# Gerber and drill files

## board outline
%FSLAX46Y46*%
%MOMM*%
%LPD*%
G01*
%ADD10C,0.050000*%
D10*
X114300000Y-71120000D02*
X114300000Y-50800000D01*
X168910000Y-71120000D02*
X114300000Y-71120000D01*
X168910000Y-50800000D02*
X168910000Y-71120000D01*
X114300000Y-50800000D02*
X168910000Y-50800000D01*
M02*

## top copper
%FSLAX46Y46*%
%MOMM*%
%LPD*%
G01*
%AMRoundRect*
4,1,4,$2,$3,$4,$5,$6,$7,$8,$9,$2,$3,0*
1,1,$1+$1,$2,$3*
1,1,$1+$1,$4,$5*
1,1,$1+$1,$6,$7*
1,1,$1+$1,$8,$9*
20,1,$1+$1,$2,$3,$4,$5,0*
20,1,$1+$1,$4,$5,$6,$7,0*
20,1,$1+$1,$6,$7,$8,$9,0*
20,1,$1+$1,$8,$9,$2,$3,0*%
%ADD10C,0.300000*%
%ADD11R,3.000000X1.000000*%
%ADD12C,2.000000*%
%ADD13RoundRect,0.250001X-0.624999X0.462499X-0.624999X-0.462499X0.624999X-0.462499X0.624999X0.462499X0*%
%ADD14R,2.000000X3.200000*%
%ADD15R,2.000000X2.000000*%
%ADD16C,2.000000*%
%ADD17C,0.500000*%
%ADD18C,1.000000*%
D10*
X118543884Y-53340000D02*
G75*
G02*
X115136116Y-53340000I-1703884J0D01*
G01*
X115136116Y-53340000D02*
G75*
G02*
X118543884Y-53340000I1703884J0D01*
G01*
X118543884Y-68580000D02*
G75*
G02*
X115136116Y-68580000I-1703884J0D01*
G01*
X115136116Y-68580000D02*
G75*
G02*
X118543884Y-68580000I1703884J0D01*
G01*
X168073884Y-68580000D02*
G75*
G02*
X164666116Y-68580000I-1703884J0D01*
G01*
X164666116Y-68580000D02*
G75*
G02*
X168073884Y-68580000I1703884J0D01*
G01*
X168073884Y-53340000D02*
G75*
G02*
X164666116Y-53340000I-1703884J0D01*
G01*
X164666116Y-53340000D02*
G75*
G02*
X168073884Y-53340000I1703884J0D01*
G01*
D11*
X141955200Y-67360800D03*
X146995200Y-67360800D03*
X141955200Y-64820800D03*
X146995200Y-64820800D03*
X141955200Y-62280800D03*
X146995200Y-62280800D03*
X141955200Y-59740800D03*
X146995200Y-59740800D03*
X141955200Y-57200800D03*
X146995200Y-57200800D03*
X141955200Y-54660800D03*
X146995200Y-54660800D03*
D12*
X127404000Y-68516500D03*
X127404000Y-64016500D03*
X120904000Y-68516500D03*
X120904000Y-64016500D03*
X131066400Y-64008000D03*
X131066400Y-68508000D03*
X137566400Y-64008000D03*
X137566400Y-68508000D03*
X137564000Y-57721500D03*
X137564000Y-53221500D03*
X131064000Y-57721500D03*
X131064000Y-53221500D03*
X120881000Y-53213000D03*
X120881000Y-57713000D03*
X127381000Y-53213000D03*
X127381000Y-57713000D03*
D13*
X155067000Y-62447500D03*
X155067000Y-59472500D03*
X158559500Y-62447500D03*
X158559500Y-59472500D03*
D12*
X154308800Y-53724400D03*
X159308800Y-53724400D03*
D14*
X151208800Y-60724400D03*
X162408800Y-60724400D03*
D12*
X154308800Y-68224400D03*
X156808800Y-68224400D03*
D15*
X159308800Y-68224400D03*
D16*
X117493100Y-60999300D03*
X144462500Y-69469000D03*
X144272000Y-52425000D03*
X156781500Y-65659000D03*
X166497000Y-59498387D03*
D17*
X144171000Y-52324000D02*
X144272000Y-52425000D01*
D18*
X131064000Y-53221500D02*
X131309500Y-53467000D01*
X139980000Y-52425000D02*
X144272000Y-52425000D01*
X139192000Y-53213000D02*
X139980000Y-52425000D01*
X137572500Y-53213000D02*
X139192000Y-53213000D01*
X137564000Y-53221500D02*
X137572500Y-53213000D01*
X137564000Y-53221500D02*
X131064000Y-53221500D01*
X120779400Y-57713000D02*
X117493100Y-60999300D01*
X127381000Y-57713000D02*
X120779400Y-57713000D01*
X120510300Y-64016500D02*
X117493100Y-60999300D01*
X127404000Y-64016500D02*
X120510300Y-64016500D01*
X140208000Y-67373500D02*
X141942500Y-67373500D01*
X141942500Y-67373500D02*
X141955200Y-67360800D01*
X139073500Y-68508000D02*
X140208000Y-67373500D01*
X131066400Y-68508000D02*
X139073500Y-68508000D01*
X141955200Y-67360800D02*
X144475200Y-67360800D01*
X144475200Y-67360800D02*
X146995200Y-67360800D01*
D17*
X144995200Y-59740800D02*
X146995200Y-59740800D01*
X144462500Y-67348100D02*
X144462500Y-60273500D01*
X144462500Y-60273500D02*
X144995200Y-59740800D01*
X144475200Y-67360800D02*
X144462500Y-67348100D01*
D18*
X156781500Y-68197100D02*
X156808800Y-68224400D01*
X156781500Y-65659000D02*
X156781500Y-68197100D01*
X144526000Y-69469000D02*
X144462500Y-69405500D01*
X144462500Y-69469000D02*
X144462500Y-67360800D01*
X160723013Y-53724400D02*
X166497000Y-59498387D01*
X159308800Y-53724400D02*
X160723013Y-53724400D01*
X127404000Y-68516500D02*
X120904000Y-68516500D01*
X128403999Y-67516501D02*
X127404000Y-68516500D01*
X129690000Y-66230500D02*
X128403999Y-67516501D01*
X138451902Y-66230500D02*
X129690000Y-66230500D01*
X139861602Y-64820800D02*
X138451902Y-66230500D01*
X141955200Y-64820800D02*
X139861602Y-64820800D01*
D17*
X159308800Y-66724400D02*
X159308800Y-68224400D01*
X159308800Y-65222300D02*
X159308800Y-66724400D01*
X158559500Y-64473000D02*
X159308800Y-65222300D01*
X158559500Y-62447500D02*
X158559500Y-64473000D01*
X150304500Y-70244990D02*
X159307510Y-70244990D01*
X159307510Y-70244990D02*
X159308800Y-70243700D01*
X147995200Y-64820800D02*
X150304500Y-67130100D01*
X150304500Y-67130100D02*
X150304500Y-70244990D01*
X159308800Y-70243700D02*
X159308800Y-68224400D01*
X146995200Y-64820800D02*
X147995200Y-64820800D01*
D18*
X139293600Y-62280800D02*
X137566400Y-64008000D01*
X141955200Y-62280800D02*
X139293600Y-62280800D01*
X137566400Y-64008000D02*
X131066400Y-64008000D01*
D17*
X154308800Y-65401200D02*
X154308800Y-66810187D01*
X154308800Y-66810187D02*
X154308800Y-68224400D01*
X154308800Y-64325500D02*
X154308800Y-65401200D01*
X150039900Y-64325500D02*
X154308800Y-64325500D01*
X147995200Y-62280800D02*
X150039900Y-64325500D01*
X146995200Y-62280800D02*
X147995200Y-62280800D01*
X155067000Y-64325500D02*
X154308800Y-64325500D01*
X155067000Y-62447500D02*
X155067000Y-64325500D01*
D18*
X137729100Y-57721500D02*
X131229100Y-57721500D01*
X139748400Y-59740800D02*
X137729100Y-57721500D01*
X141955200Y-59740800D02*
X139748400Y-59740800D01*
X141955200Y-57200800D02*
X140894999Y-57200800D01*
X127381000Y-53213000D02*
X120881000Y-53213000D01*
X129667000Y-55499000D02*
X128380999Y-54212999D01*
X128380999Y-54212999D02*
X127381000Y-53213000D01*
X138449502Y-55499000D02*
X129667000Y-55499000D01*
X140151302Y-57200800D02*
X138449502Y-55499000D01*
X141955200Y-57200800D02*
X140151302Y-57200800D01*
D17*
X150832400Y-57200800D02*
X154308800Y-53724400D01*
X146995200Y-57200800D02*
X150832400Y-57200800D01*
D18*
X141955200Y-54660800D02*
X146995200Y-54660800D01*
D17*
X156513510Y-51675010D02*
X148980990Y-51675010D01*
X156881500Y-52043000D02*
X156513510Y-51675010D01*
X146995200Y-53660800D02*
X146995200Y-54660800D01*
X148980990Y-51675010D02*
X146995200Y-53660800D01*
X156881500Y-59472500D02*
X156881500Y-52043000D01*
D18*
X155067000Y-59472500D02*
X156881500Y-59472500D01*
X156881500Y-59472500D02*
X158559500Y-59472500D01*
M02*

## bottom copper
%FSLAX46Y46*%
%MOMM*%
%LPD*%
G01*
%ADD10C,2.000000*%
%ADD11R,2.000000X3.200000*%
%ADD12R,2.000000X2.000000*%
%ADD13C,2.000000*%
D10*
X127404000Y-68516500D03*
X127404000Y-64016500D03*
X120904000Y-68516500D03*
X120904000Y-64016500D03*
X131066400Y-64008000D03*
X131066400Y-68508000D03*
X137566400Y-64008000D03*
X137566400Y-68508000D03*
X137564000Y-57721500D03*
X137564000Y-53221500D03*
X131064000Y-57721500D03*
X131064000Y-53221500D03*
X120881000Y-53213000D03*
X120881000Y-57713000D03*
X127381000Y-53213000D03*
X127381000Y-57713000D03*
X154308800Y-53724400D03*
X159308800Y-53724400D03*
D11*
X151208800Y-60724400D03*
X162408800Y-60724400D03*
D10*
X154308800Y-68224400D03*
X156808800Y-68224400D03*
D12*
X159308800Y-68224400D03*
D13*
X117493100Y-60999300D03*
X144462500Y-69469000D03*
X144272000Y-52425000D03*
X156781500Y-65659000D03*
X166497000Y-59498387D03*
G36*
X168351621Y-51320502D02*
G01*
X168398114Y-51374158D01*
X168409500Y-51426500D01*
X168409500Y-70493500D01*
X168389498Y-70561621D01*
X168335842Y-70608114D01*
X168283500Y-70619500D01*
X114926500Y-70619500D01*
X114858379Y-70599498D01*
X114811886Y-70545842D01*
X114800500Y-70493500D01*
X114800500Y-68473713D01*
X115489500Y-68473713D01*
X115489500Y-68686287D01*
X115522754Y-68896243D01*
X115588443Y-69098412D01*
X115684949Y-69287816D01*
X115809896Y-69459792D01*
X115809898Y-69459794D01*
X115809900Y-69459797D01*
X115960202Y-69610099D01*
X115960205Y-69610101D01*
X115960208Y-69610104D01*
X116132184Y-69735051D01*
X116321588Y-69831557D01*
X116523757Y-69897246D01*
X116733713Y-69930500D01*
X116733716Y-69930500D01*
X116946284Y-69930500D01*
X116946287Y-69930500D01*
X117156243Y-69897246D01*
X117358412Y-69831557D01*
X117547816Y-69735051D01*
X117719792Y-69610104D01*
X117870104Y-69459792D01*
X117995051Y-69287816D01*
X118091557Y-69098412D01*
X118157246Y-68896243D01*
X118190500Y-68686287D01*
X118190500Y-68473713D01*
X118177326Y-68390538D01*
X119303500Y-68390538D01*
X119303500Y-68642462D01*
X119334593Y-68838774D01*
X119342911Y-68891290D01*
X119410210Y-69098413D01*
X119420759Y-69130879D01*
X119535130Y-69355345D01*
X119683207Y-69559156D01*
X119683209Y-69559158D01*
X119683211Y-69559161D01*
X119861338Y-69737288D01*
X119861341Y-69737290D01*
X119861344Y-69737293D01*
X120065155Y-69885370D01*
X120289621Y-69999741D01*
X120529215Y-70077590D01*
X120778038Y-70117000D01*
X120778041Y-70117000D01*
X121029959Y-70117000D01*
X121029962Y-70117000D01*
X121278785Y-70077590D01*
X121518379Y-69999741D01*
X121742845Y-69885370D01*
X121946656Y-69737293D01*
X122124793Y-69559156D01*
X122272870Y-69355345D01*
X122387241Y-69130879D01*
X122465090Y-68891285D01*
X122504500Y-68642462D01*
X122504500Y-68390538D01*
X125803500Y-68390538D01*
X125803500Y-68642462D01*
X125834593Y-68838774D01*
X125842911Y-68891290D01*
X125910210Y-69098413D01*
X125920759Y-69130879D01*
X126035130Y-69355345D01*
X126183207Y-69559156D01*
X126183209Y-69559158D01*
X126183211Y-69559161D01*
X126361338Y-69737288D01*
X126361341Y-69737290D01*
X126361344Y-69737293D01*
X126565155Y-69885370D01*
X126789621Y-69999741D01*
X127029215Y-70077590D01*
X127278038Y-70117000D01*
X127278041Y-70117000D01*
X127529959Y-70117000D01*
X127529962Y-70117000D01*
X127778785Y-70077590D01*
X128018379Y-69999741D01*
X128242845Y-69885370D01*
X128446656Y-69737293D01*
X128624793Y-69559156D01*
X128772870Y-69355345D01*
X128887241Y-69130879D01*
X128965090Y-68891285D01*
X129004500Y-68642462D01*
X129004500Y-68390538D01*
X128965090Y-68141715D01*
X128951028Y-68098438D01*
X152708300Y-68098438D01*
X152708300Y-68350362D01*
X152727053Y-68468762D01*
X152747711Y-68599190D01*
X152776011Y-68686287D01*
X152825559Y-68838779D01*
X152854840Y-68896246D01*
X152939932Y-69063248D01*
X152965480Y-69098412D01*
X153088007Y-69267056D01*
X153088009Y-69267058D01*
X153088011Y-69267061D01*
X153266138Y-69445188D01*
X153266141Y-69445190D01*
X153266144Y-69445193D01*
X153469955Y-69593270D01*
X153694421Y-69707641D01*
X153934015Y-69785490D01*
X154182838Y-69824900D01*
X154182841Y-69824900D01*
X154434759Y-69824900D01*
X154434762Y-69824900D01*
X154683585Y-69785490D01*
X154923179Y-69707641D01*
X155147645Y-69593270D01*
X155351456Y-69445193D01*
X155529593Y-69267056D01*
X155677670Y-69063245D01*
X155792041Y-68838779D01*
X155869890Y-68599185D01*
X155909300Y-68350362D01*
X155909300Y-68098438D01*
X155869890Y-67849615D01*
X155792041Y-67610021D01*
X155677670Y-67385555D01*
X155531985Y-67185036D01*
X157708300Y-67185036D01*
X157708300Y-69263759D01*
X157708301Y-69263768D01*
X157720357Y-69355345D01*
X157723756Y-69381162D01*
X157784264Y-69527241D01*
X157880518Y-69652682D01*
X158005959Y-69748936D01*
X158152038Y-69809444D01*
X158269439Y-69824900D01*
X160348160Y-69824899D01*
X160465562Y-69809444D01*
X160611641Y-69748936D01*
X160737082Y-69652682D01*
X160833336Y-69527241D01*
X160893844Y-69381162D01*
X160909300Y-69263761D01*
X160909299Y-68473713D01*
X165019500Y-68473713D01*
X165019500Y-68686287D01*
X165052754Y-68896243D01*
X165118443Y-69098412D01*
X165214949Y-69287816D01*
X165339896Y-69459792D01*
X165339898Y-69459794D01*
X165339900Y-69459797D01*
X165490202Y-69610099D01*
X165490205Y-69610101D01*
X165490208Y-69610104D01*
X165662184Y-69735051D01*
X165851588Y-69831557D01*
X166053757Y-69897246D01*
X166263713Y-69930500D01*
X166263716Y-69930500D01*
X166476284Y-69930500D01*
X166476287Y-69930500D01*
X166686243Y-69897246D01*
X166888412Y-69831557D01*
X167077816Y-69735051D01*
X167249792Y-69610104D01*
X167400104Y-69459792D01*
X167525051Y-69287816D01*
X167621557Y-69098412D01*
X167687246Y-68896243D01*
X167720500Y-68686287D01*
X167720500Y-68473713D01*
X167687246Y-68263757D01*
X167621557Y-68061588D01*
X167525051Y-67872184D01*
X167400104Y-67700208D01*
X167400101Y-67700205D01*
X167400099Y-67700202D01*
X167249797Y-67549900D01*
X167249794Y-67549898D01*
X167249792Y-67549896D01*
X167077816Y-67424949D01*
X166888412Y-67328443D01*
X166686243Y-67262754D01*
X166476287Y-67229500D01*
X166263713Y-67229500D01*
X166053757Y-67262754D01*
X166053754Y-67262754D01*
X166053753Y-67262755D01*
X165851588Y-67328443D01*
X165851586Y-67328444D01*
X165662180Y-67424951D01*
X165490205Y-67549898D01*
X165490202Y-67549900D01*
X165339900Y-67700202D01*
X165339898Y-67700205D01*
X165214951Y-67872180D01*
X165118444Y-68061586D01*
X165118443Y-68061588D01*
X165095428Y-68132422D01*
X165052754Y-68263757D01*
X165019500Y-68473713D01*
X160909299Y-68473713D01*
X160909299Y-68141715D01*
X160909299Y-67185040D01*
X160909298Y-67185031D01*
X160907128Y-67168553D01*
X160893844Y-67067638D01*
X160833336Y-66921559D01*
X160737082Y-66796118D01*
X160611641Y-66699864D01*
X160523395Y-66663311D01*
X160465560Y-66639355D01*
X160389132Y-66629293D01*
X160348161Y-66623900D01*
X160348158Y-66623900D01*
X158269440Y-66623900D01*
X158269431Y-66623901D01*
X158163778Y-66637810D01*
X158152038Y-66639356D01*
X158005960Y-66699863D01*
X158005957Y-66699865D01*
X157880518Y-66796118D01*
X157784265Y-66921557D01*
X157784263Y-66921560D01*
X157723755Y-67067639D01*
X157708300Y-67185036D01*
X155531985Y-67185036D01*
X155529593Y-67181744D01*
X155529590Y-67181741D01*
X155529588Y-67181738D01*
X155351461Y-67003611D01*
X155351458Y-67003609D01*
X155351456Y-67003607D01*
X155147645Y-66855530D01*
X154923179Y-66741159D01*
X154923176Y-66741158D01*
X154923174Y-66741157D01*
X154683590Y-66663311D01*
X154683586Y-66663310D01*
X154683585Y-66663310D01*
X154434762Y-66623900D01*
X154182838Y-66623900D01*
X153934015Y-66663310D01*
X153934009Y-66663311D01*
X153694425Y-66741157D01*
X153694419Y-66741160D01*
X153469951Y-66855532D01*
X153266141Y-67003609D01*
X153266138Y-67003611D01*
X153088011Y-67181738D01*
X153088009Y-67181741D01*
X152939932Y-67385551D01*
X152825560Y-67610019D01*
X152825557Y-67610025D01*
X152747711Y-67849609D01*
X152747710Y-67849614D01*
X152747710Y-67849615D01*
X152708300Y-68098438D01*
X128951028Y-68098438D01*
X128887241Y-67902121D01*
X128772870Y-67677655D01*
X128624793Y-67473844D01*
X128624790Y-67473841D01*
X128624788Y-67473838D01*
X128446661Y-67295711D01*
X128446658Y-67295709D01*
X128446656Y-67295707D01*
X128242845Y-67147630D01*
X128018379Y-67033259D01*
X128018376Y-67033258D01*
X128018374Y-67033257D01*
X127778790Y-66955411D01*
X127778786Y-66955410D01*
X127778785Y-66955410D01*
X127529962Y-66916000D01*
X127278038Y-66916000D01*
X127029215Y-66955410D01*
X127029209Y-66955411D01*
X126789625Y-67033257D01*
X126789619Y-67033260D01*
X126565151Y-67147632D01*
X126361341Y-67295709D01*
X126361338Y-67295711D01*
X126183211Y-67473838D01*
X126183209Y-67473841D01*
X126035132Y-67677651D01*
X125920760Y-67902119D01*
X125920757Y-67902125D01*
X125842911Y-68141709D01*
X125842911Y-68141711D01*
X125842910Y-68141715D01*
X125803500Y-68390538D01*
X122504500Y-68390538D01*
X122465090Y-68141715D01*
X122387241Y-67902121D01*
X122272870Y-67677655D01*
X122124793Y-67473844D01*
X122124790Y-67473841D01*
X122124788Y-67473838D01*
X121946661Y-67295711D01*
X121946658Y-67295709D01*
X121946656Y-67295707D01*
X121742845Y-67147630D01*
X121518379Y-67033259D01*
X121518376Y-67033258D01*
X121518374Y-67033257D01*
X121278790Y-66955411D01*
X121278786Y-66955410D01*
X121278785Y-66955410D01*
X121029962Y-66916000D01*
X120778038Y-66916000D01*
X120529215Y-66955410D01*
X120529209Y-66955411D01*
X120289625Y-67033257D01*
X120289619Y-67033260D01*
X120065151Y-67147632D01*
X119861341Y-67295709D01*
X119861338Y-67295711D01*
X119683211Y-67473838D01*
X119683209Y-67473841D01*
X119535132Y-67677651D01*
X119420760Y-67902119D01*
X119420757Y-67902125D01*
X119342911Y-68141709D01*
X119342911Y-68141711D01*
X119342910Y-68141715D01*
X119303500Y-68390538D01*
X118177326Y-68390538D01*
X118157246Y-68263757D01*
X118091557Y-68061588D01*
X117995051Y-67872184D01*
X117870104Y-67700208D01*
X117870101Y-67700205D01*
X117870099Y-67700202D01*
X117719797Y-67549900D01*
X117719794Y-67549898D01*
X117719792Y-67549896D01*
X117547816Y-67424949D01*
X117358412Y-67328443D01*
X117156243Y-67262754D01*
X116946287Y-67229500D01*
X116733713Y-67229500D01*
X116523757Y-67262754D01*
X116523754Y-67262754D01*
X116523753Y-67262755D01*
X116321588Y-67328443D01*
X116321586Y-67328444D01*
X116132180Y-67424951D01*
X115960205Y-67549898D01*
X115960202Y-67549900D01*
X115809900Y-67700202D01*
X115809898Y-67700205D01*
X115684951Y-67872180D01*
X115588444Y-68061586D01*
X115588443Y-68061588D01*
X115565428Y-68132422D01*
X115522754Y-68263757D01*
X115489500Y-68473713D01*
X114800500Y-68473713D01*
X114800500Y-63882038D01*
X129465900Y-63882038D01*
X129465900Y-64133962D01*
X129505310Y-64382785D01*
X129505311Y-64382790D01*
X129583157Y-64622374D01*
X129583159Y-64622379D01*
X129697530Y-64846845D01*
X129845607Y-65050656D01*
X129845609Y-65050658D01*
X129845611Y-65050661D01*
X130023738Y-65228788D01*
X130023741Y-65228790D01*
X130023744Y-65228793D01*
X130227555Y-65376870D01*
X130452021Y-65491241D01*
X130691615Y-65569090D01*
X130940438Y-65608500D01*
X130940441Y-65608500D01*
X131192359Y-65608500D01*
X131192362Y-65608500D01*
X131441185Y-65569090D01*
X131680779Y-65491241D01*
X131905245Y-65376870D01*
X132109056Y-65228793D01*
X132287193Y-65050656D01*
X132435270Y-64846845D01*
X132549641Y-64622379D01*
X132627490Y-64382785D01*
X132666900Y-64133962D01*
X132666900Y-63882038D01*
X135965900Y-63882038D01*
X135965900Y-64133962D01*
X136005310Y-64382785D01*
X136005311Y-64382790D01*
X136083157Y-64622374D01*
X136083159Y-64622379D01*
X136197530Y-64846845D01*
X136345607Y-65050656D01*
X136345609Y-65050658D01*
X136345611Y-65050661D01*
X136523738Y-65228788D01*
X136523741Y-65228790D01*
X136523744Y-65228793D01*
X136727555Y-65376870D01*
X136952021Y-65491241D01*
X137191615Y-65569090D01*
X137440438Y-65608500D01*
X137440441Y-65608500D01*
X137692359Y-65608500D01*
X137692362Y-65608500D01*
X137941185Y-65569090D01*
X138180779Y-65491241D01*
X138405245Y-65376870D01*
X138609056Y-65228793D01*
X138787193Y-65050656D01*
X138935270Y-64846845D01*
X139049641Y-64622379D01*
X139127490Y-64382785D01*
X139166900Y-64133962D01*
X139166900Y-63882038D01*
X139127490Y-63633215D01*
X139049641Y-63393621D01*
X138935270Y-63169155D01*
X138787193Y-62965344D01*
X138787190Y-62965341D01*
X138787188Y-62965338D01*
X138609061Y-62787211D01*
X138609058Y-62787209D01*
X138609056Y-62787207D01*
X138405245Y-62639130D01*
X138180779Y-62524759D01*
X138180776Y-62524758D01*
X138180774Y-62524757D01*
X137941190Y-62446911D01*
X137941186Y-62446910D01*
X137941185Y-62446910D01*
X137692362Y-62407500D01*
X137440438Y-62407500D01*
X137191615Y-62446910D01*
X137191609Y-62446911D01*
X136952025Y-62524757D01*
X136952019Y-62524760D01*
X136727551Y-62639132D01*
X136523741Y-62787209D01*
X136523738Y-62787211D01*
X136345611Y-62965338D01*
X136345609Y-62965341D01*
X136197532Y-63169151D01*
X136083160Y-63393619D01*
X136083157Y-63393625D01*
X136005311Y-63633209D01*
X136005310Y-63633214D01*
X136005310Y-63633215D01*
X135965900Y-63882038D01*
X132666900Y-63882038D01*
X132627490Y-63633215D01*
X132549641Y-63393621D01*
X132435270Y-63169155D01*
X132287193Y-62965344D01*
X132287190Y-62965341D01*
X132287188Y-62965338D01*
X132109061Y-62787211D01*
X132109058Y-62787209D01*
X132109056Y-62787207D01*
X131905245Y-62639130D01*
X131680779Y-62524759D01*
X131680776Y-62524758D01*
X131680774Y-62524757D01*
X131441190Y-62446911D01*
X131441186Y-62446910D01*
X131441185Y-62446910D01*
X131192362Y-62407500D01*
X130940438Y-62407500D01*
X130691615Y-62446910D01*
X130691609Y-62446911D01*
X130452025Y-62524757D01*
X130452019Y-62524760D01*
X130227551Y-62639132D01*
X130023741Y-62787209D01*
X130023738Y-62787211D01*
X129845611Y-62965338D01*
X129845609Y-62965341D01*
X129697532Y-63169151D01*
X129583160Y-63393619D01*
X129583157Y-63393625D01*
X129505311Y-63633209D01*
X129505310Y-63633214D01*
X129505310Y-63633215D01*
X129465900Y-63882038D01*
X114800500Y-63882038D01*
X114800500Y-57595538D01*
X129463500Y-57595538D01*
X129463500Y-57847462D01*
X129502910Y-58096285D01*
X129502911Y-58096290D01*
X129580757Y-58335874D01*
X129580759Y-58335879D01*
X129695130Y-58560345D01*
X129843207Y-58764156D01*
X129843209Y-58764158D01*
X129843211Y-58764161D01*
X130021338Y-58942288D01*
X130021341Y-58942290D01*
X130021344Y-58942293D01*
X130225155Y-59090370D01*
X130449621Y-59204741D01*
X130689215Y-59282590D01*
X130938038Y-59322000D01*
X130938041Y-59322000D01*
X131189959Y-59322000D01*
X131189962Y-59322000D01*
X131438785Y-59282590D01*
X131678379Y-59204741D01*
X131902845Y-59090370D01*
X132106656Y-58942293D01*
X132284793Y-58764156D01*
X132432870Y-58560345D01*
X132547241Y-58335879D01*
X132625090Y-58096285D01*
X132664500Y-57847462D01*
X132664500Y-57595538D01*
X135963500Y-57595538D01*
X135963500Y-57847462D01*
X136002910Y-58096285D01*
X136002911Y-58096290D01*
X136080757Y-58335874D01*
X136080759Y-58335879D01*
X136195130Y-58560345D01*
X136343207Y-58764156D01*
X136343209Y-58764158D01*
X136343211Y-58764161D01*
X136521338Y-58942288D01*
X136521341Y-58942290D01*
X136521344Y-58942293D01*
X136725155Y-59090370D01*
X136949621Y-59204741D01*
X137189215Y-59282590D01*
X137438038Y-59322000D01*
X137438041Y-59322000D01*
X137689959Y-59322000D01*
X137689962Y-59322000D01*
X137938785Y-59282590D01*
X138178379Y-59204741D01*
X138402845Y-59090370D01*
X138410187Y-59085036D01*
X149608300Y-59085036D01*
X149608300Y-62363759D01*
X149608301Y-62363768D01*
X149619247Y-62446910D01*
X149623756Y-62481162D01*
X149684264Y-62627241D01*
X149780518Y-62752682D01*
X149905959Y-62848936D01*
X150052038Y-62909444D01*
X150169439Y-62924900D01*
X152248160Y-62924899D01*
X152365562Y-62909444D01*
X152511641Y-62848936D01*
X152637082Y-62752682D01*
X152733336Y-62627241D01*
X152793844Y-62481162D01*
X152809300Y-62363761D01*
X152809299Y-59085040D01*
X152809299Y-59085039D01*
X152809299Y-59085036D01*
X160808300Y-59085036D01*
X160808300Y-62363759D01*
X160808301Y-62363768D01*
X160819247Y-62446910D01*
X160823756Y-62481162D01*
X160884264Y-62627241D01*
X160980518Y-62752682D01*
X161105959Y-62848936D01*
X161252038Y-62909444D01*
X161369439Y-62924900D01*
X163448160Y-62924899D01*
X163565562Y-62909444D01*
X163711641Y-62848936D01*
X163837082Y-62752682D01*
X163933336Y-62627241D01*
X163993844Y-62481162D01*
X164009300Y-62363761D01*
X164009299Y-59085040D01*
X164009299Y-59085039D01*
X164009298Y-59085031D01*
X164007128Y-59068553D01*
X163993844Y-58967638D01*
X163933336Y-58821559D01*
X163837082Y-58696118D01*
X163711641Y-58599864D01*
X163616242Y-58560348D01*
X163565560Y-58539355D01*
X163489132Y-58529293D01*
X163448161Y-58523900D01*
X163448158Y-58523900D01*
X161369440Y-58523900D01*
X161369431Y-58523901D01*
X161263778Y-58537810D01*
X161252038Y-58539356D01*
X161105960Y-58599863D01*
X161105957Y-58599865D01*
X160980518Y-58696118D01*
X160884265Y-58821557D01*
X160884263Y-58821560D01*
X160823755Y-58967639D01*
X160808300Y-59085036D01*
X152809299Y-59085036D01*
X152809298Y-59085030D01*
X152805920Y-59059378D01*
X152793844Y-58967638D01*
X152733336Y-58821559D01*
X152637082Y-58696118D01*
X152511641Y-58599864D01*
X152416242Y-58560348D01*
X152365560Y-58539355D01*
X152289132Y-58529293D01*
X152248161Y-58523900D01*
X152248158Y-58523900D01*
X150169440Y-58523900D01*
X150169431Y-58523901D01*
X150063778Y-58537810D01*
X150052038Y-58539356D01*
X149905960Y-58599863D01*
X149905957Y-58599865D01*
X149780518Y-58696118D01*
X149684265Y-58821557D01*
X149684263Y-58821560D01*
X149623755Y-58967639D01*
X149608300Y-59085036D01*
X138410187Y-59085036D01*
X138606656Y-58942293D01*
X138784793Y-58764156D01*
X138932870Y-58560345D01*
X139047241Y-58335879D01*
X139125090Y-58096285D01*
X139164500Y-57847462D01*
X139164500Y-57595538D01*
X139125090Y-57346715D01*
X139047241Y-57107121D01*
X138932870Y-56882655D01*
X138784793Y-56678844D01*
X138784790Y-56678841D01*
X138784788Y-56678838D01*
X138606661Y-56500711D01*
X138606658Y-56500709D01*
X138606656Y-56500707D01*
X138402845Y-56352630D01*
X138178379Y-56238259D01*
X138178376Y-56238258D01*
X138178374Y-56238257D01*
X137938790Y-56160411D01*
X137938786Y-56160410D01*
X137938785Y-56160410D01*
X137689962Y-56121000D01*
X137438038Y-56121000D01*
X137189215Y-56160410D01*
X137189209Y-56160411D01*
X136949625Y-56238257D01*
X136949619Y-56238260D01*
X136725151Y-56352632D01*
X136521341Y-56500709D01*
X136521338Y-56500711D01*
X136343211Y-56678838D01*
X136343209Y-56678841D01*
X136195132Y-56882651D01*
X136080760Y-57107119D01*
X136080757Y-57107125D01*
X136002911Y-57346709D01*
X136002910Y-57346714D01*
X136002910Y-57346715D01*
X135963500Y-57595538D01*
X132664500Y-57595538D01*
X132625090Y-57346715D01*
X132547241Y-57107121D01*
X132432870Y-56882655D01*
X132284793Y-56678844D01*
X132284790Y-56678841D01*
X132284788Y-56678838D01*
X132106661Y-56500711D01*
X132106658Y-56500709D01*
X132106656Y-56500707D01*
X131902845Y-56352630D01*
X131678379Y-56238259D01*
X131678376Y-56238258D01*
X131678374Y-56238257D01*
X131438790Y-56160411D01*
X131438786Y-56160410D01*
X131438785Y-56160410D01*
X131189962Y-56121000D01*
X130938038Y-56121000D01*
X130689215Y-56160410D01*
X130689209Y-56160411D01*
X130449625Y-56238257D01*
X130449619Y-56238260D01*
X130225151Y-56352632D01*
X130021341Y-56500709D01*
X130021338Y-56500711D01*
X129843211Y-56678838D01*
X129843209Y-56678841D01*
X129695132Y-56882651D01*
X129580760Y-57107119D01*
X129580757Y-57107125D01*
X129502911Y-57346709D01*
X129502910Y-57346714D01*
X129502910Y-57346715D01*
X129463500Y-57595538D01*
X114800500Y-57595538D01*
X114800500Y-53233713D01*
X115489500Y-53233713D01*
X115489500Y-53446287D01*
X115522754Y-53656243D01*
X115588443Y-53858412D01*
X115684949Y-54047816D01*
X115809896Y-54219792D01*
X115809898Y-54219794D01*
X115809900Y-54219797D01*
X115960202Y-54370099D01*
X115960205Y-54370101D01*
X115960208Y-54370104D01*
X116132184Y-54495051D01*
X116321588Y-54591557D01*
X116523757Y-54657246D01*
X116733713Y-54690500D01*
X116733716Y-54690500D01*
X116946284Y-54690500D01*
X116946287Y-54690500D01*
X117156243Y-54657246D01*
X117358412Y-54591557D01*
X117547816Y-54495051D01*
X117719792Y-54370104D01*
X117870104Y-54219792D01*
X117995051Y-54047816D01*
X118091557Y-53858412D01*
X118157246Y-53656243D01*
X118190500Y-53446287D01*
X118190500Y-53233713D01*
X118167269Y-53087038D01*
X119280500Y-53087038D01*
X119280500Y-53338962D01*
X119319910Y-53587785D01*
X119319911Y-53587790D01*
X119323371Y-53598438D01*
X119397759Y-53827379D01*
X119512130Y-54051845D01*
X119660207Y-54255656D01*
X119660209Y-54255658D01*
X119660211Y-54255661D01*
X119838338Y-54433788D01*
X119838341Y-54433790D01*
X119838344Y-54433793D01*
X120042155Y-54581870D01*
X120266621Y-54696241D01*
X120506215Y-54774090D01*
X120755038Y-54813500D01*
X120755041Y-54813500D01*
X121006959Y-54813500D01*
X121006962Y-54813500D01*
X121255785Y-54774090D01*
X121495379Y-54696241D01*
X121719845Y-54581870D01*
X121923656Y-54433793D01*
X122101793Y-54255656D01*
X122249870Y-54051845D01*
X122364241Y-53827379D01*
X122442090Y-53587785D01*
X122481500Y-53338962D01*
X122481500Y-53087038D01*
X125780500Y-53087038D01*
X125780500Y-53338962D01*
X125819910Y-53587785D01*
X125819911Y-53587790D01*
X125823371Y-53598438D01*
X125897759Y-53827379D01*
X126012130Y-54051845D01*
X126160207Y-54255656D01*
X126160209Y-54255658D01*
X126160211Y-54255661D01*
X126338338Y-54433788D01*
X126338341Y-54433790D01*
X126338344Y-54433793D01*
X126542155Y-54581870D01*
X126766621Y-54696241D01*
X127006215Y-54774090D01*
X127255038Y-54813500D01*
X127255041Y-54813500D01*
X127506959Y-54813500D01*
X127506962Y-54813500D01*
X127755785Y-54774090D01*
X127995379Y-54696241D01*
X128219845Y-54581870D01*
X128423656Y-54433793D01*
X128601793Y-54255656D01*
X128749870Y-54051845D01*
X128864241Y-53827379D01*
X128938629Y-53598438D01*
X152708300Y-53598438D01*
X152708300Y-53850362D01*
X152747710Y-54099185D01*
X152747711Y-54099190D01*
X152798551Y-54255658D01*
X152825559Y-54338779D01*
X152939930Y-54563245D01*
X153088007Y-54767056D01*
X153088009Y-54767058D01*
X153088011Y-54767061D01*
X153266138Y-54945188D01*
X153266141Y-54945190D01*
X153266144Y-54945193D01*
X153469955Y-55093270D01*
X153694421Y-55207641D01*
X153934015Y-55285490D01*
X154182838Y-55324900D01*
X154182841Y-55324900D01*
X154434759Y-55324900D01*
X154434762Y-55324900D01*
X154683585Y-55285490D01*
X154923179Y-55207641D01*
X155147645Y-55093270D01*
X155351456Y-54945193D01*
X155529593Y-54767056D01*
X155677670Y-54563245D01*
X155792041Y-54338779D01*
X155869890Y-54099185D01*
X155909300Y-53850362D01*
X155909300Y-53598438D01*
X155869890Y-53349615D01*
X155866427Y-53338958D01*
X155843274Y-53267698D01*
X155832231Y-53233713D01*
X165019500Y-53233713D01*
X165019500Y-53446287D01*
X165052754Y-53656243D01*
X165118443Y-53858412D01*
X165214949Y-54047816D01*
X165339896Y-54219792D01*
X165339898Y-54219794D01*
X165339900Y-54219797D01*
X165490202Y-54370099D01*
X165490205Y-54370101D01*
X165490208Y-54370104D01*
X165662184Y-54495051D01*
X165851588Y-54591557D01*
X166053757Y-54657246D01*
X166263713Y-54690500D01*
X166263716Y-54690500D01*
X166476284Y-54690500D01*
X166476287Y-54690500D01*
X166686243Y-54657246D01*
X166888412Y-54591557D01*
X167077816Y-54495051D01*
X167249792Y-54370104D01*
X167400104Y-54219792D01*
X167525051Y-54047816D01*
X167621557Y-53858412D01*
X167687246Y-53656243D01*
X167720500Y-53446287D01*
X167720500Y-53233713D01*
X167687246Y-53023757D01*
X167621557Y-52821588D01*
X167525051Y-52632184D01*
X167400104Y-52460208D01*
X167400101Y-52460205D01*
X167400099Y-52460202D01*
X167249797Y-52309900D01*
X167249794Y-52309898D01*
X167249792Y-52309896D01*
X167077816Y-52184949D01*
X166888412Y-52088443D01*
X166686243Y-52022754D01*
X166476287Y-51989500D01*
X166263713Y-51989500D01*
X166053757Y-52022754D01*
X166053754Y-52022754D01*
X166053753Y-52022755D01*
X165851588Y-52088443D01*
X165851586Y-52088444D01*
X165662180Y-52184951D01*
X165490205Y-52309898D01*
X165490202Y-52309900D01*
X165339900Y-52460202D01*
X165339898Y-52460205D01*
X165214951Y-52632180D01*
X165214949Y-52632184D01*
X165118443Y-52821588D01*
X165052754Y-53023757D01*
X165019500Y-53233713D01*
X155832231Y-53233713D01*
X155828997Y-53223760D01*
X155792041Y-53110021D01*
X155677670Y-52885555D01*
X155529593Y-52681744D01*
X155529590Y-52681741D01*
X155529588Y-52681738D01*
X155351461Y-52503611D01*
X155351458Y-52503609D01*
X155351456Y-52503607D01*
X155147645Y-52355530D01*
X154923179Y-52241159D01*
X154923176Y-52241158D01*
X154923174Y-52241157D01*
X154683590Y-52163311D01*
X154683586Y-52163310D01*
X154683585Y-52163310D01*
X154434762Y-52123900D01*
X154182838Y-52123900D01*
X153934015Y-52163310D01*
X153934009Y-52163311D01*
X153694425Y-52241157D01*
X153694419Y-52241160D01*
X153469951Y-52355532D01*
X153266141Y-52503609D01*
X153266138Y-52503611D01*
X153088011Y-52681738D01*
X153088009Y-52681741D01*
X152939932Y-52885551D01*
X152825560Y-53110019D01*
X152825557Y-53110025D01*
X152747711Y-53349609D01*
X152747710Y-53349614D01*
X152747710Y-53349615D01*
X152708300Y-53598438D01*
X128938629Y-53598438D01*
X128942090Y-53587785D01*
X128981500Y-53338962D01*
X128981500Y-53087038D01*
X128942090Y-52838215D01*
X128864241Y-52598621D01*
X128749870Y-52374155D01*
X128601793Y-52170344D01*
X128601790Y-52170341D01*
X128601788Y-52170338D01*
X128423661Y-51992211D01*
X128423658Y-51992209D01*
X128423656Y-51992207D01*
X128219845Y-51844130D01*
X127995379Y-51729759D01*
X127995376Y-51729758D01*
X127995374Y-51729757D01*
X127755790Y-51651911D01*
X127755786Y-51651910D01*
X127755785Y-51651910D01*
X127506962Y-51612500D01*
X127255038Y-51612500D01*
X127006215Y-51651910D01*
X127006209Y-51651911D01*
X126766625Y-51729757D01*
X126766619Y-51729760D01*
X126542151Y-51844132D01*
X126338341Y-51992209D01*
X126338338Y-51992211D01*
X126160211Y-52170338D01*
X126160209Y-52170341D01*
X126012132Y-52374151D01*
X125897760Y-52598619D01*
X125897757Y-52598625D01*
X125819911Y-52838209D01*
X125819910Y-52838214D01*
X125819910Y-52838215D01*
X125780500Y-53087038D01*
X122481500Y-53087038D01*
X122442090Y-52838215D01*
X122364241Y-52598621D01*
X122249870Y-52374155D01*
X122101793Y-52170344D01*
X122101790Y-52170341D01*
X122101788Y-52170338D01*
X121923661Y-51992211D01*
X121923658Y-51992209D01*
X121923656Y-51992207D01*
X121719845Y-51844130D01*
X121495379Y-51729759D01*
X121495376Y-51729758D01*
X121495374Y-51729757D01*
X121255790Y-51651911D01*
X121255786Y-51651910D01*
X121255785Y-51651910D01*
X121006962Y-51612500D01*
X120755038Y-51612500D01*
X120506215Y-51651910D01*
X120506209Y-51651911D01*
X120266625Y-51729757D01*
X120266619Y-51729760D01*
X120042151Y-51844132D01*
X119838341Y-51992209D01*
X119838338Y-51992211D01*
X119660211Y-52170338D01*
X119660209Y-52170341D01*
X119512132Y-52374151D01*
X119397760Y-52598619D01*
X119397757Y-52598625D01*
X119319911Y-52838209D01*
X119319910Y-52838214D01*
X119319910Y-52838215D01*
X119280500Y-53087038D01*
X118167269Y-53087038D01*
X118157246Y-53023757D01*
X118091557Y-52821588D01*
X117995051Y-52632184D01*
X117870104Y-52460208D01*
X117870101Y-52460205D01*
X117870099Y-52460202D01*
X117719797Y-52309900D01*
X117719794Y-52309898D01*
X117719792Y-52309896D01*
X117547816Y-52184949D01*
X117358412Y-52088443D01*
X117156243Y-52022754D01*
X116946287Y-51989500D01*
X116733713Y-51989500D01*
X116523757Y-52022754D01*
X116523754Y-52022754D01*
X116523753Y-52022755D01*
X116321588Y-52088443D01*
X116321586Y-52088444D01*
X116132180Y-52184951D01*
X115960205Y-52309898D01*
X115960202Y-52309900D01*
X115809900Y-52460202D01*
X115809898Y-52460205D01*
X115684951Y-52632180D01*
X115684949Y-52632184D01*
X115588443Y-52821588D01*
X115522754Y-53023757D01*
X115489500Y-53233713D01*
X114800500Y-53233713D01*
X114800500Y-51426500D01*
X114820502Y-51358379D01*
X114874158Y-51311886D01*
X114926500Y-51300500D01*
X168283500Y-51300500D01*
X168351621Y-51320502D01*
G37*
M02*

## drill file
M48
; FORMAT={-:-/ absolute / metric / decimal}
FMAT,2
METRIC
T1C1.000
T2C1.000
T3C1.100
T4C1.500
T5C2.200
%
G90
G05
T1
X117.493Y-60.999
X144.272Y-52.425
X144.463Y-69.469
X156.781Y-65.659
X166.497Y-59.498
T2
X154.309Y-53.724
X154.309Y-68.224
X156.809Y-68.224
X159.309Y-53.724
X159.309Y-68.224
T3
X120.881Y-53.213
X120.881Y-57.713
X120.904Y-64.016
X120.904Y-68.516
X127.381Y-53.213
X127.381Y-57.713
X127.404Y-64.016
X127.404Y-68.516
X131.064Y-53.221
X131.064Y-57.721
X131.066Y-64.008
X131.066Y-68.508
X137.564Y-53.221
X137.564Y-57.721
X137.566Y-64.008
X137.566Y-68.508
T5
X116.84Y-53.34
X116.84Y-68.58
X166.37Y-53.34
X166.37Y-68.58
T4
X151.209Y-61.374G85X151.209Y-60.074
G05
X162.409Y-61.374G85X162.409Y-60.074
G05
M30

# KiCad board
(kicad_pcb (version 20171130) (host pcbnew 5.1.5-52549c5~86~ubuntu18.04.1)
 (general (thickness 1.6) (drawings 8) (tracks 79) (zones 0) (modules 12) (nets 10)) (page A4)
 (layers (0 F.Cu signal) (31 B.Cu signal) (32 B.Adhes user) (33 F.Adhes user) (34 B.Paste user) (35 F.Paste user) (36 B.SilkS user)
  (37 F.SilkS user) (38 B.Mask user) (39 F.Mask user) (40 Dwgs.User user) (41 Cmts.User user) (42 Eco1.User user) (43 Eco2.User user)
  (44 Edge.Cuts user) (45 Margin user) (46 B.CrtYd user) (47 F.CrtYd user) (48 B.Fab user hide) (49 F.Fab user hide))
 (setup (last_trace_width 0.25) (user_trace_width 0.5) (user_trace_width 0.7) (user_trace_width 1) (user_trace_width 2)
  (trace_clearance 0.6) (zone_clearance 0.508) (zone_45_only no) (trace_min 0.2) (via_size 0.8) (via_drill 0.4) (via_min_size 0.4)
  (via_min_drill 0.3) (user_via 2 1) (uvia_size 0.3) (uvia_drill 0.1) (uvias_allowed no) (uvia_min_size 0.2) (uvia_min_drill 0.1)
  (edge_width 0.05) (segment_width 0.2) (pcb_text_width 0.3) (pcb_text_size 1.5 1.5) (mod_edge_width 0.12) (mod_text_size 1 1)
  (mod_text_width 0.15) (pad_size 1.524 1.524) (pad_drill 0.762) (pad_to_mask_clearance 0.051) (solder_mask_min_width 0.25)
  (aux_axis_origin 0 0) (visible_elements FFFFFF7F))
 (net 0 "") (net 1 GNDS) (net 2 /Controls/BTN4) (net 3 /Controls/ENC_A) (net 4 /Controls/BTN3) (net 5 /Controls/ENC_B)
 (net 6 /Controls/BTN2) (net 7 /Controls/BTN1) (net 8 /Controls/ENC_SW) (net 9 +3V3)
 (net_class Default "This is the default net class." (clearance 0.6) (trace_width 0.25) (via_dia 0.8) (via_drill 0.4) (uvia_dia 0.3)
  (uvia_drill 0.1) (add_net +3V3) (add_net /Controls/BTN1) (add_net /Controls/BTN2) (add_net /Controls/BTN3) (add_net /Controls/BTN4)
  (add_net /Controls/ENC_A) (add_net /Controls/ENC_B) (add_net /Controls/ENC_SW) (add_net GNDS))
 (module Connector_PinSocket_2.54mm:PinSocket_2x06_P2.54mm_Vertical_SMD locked (layer F.Cu) (at 144.4752 61.0108)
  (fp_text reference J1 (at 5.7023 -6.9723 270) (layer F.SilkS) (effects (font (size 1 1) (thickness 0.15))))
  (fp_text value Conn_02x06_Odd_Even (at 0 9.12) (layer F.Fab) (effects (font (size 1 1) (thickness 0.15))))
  (pad 12 smd rect (at -2.52 6.35) (size 3 1) (layers F.Cu F.Paste F.Mask) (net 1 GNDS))
  (pad 11 smd rect (at 2.52 6.35) (size 3 1) (layers F.Cu F.Paste F.Mask) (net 1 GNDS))
  (pad 10 smd rect (at -2.52 3.81) (size 3 1) (layers F.Cu F.Paste F.Mask) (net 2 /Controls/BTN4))
  (pad 9 smd rect (at 2.52 3.81) (size 3 1) (layers F.Cu F.Paste F.Mask) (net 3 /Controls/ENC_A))
  (pad 8 smd rect (at -2.52 1.27) (size 3 1) (layers F.Cu F.Paste F.Mask) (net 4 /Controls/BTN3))
  (pad 7 smd rect (at 2.52 1.27) (size 3 1) (layers F.Cu F.Paste F.Mask) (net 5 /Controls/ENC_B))
  (pad 6 smd rect (at -2.52 -1.27) (size 3 1) (layers F.Cu F.Paste F.Mask) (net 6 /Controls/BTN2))
  (pad 5 smd rect (at 2.52 -1.27) (size 3 1) (layers F.Cu F.Paste F.Mask) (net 1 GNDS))
  (pad 4 smd rect (at -2.52 -3.81) (size 3 1) (layers F.Cu F.Paste F.Mask) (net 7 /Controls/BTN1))
  (pad 3 smd rect (at 2.52 -3.81) (size 3 1) (layers F.Cu F.Paste F.Mask) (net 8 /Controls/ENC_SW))
  (pad 2 smd rect (at -2.52 -6.35) (size 3 1) (layers F.Cu F.Paste F.Mask) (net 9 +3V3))
  (pad 1 smd rect (at 2.52 -6.35) (size 3 1) (layers F.Cu F.Paste F.Mask) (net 9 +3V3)))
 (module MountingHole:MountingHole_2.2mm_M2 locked (layer F.Cu) (at 166.37 53.34)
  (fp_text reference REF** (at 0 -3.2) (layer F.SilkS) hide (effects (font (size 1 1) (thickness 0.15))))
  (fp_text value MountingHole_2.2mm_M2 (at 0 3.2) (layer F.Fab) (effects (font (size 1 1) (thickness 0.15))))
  (pad 1 np_thru_hole circle (at 0 0) (size 2.2 2.2) (drill 2.2) (layers *.Cu *.Mask)))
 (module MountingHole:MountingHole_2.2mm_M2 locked (layer F.Cu) (at 166.37 68.58)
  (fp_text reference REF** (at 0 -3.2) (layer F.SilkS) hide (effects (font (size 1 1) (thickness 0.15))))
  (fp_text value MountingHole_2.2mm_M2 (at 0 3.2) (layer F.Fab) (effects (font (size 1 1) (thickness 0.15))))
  (pad 1 np_thru_hole circle (at 0 0) (size 2.2 2.2) (drill 2.2) (layers *.Cu *.Mask)))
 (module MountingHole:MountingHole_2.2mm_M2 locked (layer F.Cu) (at 116.84 68.58)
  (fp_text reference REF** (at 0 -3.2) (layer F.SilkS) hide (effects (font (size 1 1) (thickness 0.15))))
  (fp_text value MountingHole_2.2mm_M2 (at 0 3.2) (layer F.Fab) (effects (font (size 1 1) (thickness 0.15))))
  (pad 1 np_thru_hole circle (at 0 0) (size 2.2 2.2) (drill 2.2) (layers *.Cu *.Mask)))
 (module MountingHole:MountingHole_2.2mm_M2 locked (layer F.Cu) (at 116.84 53.34)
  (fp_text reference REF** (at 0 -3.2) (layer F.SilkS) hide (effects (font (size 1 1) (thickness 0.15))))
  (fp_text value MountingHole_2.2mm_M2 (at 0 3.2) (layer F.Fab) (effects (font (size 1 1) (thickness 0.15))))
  (pad 1 np_thru_hole circle (at 0 0) (size 2.2 2.2) (drill 2.2) (layers *.Cu *.Mask)))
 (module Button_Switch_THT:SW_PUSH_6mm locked (layer B.Cu) (at 120.904 68.5165)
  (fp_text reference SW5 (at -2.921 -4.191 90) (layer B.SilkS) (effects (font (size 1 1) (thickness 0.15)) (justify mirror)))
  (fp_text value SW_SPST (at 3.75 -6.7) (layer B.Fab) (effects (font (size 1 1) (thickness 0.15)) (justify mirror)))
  (pad 1 thru_hole circle (at 6.5 0 270) (size 2 2) (drill 1.1) (layers *.Cu *.Mask) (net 2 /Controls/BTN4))
  (pad 2 thru_hole circle (at 6.5 -4.5 270) (size 2 2) (drill 1.1) (layers *.Cu *.Mask) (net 1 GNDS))
  (pad 1 thru_hole circle (at 0 0 270) (size 2 2) (drill 1.1) (layers *.Cu *.Mask) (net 2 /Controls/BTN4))
  (pad 2 thru_hole circle (at 0 -4.5 270) (size 2 2) (drill 1.1) (layers *.Cu *.Mask) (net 1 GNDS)))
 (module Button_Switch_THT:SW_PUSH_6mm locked (layer B.Cu) (at 137.5664 64.008 180)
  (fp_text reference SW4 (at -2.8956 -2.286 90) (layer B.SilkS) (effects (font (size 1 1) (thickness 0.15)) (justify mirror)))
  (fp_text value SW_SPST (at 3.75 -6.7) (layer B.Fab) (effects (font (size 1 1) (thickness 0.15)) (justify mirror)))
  (pad 1 thru_hole circle (at 6.5 0 90) (size 2 2) (drill 1.1) (layers *.Cu *.Mask) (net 4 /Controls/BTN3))
  (pad 2 thru_hole circle (at 6.5 -4.5 90) (size 2 2) (drill 1.1) (layers *.Cu *.Mask) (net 1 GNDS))
  (pad 1 thru_hole circle (at 0 0 90) (size 2 2) (drill 1.1) (layers *.Cu *.Mask) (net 4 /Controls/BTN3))
  (pad 2 thru_hole circle (at 0 -4.5 90) (size 2 2) (drill 1.1) (layers *.Cu *.Mask) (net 1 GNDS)))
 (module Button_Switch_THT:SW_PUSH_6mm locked (layer B.Cu) (at 131.064 57.7215)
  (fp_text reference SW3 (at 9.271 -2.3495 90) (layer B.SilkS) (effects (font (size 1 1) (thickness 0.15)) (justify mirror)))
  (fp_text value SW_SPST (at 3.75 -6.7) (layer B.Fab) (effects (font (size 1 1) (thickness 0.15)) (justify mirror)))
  (pad 1 thru_hole circle (at 6.5 0 270) (size 2 2) (drill 1.1) (layers *.Cu *.Mask) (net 6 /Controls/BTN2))
  (pad 2 thru_hole circle (at 6.5 -4.5 270) (size 2 2) (drill 1.1) (layers *.Cu *.Mask) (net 1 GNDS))
  (pad 1 thru_hole circle (at 0 0 270) (size 2 2) (drill 1.1) (layers *.Cu *.Mask) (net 6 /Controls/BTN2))
  (pad 2 thru_hole circle (at 0 -4.5 270) (size 2 2) (drill 1.1) (layers *.Cu *.Mask) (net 1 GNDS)))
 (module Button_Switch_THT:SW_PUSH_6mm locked (layer B.Cu) (at 127.381 53.213 180)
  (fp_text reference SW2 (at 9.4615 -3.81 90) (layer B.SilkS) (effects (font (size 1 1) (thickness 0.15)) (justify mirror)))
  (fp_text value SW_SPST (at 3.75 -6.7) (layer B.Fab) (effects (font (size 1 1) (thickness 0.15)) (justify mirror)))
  (pad 1 thru_hole circle (at 6.5 0 90) (size 2 2) (drill 1.1) (layers *.Cu *.Mask) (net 7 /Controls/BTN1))
  (pad 2 thru_hole circle (at 6.5 -4.5 90) (size 2 2) (drill 1.1) (layers *.Cu *.Mask) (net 1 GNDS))
  (pad 1 thru_hole circle (at 0 0 90) (size 2 2) (drill 1.1) (layers *.Cu *.Mask) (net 7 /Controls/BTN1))
  (pad 2 thru_hole circle (at 0 -4.5 90) (size 2 2) (drill 1.1) (layers *.Cu *.Mask) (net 1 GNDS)))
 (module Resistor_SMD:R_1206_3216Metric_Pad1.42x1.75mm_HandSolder (layer F.Cu) (at 155.067 60.96 270)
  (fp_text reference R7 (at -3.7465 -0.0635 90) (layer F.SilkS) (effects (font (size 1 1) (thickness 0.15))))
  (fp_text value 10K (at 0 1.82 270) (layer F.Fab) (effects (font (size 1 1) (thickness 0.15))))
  (pad 2 smd roundrect (at 1.4875 0 270) (size 1.425 1.75) (layers F.Cu F.Paste F.Mask) (roundrect_rratio 0.175439) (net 5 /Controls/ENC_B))
  (pad 1 smd roundrect (at -1.4875 0 270) (size 1.425 1.75) (layers F.Cu F.Paste F.Mask) (roundrect_rratio 0.175439) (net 9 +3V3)))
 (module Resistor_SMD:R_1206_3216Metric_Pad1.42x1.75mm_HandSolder (layer F.Cu) (at 158.5595 60.96 270)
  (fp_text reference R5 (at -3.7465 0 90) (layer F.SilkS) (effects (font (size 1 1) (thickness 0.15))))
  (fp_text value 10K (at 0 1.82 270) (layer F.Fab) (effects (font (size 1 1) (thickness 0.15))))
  (pad 2 smd roundrect (at 1.4875 0 270) (size 1.425 1.75) (layers F.Cu F.Paste F.Mask) (roundrect_rratio 0.175439) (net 3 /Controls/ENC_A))
  (pad 1 smd roundrect (at -1.4875 0 270) (size 1.425 1.75) (layers F.Cu F.Paste F.Mask) (roundrect_rratio 0.175439) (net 9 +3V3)))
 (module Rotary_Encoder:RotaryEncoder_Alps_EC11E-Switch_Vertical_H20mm (layer B.Cu) (at 159.3088 68.2244 90)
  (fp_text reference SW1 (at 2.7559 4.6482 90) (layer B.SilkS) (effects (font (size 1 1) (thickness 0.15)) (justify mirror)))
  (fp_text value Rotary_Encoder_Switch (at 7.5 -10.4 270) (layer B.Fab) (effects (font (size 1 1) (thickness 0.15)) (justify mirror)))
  (pad S1 thru_hole circle (at 14.5 -5 90) (size 2 2) (drill 1) (layers *.Cu *.Mask) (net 8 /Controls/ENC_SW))
  (pad S2 thru_hole circle (at 14.5 0 90) (size 2 2) (drill 1) (layers *.Cu *.Mask) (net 1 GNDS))
  (pad MP thru_hole rect (at 7.5 -8.1 90) (size 3.2 2) (drill oval 2.8 1.5) (layers *.Cu *.Mask))
  (pad MP thru_hole rect (at 7.5 3.1 90) (size 3.2 2) (drill oval 2.8 1.5) (layers *.Cu *.Mask))
  (pad B thru_hole circle (at 0 -5 90) (size 2 2) (drill 1) (layers *.Cu *.Mask) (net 5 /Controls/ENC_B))
  (pad C thru_hole circle (at 0 -2.5 90) (size 2 2) (drill 1) (layers *.Cu *.Mask) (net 1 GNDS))
  (pad A thru_hole rect (at 0 0 90) (size 2 2) (drill 1) (layers *.Cu *.Mask) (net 3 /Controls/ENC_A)))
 (gr_circle (center 116.84 53.34) (end 118.543884 53.34) (layer F.Cu) (width 0.3))
 (gr_circle (center 116.84 68.58) (end 118.543884 68.58) (layer F.Cu) (width 0.3))
 (gr_circle (center 166.37 68.58) (end 168.073884 68.58) (layer F.Cu) (width 0.3))
 (gr_circle (center 166.37 53.34) (end 168.073884 53.34) (layer F.Cu) (width 0.3))
 (gr_line (start 114.3 71.12) (end 114.3 50.8) (layer Edge.Cuts) (width 0.05))
 (gr_line (start 168.91 71.12) (end 114.3 71.12) (layer Edge.Cuts) (width 0.05))
 (gr_line (start 168.91 50.8) (end 168.91 71.12) (layer Edge.Cuts) (width 0.05))
 (gr_line (start 114.3 50.8) (end 168.91 50.8) (layer Edge.Cuts) (width 0.05))
 (via (at 117.4931 60.9993) (size 2) (drill 1) (layers F.Cu B.Cu) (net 1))
 (via (at 144.4625 69.469) (size 2) (drill 1) (layers F.Cu B.Cu) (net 1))
 (via (at 144.272 52.425) (size 2) (drill 1) (layers F.Cu B.Cu) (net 1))
 (segment (start 144.171 52.324) (end 144.272 52.425) (width 0.5) (layer F.Cu) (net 1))
 (segment (start 131.064 53.2215) (end 131.3095 53.467) (width 1) (layer F.Cu) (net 1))
 (segment (start 139.98 52.425) (end 144.272 52.425) (width 1) (layer F.Cu) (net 1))
 (segment (start 139.192 53.213) (end 139.98 52.425) (width 1) (layer F.Cu) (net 1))
 (segment (start 137.5725 53.213) (end 139.192 53.213) (width 1) (layer F.Cu) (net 1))
 (segment (start 137.564 53.2215) (end 137.5725 53.213) (width 1) (layer F.Cu) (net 1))
 (segment (start 137.564 53.2215) (end 131.064 53.2215) (width 1) (layer F.Cu) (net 1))
 (segment (start 120.7794 57.713) (end 117.4931 60.9993) (width 1) (layer F.Cu) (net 1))
 (segment (start 127.381 57.713) (end 120.7794 57.713) (width 1) (layer F.Cu) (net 1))
 (segment (start 120.5103 64.0165) (end 117.4931 60.9993) (width 1) (layer F.Cu) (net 1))
 (segment (start 127.404 64.0165) (end 120.5103 64.0165) (width 1) (layer F.Cu) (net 1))
 (segment (start 140.208 67.3735) (end 141.9425 67.3735) (width 1) (layer F.Cu) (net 1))
 (segment (start 141.9425 67.3735) (end 141.9552 67.3608) (width 1) (layer F.Cu) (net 1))
 (segment (start 139.0735 68.508) (end 140.208 67.3735) (width 1) (layer F.Cu) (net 1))
 (segment (start 131.0664 68.508) (end 139.0735 68.508) (width 1) (layer F.Cu) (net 1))
 (segment (start 141.9552 67.3608) (end 144.4752 67.3608) (width 1) (layer F.Cu) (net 1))
 (segment (start 144.4752 67.3608) (end 146.9952 67.3608) (width 1) (layer F.Cu) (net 1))
 (segment (start 144.9952 59.7408) (end 146.9952 59.7408) (width 0.5) (layer F.Cu) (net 1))
 (segment (start 144.4625 67.3481) (end 144.4625 60.2735) (width 0.5) (layer F.Cu) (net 1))
 (segment (start 144.4625 60.2735) (end 144.9952 59.7408) (width 0.5) (layer F.Cu) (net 1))
 (segment (start 144.4752 67.3608) (end 144.4625 67.3481) (width 0.5) (layer F.Cu) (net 1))
 (via (at 156.7815 65.659) (size 2) (drill 1) (layers F.Cu B.Cu) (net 1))
 (segment (start 156.7815 68.1971) (end 156.8088 68.2244) (width 1) (layer F.Cu) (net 1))
 (segment (start 156.7815 65.659) (end 156.7815 68.1971) (width 1) (layer F.Cu) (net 1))
 (segment (start 144.526 69.469) (end 144.4625 69.4055) (width 1) (layer F.Cu) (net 1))
 (segment (start 144.4625 69.469) (end 144.4625 67.3608) (width 1) (layer F.Cu) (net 1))
 (segment (start 160.723013 53.7244) (end 166.497 59.498387) (width 1) (layer F.Cu) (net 1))
 (segment (start 159.3088 53.7244) (end 160.723013 53.7244) (width 1) (layer F.Cu) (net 1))
 (via (at 166.497 59.498387) (size 2) (drill 1) (layers F.Cu B.Cu) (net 1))
 (segment (start 127.404 68.5165) (end 120.904 68.5165) (width 1) (layer F.Cu) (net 2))
 (segment (start 128.403999 67.516501) (end 127.404 68.5165) (width 1) (layer F.Cu) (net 2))
 (segment (start 129.69 66.2305) (end 128.403999 67.516501) (width 1) (layer F.Cu) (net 2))
 (segment (start 138.451902 66.2305) (end 129.69 66.2305) (width 1) (layer F.Cu) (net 2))
 (segment (start 139.861602 64.8208) (end 138.451902 66.2305) (width 1) (layer F.Cu) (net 2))
 (segment (start 141.9552 64.8208) (end 139.861602 64.8208) (width 1) (layer F.Cu) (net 2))
 (segment (start 159.3088 66.7244) (end 159.3088 68.2244) (width 0.5) (layer F.Cu) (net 3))
 (segment (start 159.3088 65.2223) (end 159.3088 66.7244) (width 0.5) (layer F.Cu) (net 3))
 (segment (start 158.5595 64.473) (end 159.3088 65.2223) (width 0.5) (layer F.Cu) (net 3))
 (segment (start 158.5595 62.4475) (end 158.5595 64.473) (width 0.5) (layer F.Cu) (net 3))
 (segment (start 150.3045 70.24499) (end 159.30751 70.24499) (width 0.5) (layer F.Cu) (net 3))
 (segment (start 159.30751 70.24499) (end 159.3088 70.2437) (width 0.5) (layer F.Cu) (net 3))
 (segment (start 147.9952 64.8208) (end 150.3045 67.1301) (width 0.5) (layer F.Cu) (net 3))
 (segment (start 150.3045 67.1301) (end 150.3045 70.24499) (width 0.5) (layer F.Cu) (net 3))
 (segment (start 159.3088 70.2437) (end 159.3088 68.2244) (width 0.5) (layer F.Cu) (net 3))
 (segment (start 146.9952 64.8208) (end 147.9952 64.8208) (width 0.5) (layer F.Cu) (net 3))
 (segment (start 139.2936 62.2808) (end 137.5664 64.008) (width 1) (layer F.Cu) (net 4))
 (segment (start 141.9552 62.2808) (end 139.2936 62.2808) (width 1) (layer F.Cu) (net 4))
 (segment (start 137.5664 64.008) (end 131.0664 64.008) (width 1) (layer F.Cu) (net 4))
 (segment (start 154.3088 65.4012) (end 154.3088 66.810187) (width 0.5) (layer F.Cu) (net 5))
 (segment (start 154.3088 66.810187) (end 154.3088 68.2244) (width 0.5) (layer F.Cu) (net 5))
 (segment (start 154.3088 64.3255) (end 154.3088 65.4012) (width 0.5) (layer F.Cu) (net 5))
 (segment (start 150.0399 64.3255) (end 154.3088 64.3255) (width 0.5) (layer F.Cu) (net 5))
 (segment (start 147.9952 62.2808) (end 150.0399 64.3255) (width 0.5) (layer F.Cu) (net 5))
 (segment (start 146.9952 62.2808) (end 147.9952 62.2808) (width 0.5) (layer F.Cu) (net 5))
 (segment (start 155.067 64.3255) (end 154.3088 64.3255) (width 0.5) (layer F.Cu) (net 5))
 (segment (start 155.067 62.4475) (end 155.067 64.3255) (width 0.5) (layer F.Cu) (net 5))
 (segment (start 137.7291 57.7215) (end 131.2291 57.7215) (width 1) (layer F.Cu) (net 6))
 (segment (start 139.7484 59.7408) (end 137.7291 57.7215) (width 1) (layer F.Cu) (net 6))
 (segment (start 141.9552 59.7408) (end 139.7484 59.7408) (width 1) (layer F.Cu) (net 6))
 (segment (start 141.9552 57.2008) (end 140.894999 57.2008) (width 1) (layer F.Cu) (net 7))
 (segment (start 127.381 53.213) (end 120.881 53.213) (width 1) (layer F.Cu) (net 7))
 (segment (start 129.667 55.499) (end 128.380999 54.212999) (width 1) (layer F.Cu) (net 7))
 (segment (start 128.380999 54.212999) (end 127.381 53.213) (width 1) (layer F.Cu) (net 7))
 (segment (start 138.449502 55.499) (end 129.667 55.499) (width 1) (layer F.Cu) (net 7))
 (segment (start 140.151302 57.2008) (end 138.449502 55.499) (width 1) (layer F.Cu) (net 7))
 (segment (start 141.9552 57.2008) (end 140.151302 57.2008) (width 1) (layer F.Cu) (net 7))
 (segment (start 150.8324 57.2008) (end 154.3088 53.7244) (width 0.5) (layer F.Cu) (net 8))
 (segment (start 146.9952 57.2008) (end 150.8324 57.2008) (width 0.5) (layer F.Cu) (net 8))
 (segment (start 141.9552 54.6608) (end 146.9952 54.6608) (width 1) (layer F.Cu) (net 9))
 (segment (start 156.51351 51.67501) (end 148.98099 51.67501) (width 0.5) (layer F.Cu) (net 9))
 (segment (start 156.8815 52.043) (end 156.51351 51.67501) (width 0.5) (layer F.Cu) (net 9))
 (segment (start 146.9952 53.6608) (end 146.9952 54.6608) (width 0.5) (layer F.Cu) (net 9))
 (segment (start 148.98099 51.67501) (end 146.9952 53.6608) (width 0.5) (layer F.Cu) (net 9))
 (segment (start 156.8815 59.4725) (end 156.8815 52.043) (width 0.5) (layer F.Cu) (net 9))
 (segment (start 155.067 59.4725) (end 156.8815 59.4725) (width 1) (layer F.Cu) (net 9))
 (segment (start 156.8815 59.4725) (end 158.5595 59.4725) (width 1) (layer F.Cu) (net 9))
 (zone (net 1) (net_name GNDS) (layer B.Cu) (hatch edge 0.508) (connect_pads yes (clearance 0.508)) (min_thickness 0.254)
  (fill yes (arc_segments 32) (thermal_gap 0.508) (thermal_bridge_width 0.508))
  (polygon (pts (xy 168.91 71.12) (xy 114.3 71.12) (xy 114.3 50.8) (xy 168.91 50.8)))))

